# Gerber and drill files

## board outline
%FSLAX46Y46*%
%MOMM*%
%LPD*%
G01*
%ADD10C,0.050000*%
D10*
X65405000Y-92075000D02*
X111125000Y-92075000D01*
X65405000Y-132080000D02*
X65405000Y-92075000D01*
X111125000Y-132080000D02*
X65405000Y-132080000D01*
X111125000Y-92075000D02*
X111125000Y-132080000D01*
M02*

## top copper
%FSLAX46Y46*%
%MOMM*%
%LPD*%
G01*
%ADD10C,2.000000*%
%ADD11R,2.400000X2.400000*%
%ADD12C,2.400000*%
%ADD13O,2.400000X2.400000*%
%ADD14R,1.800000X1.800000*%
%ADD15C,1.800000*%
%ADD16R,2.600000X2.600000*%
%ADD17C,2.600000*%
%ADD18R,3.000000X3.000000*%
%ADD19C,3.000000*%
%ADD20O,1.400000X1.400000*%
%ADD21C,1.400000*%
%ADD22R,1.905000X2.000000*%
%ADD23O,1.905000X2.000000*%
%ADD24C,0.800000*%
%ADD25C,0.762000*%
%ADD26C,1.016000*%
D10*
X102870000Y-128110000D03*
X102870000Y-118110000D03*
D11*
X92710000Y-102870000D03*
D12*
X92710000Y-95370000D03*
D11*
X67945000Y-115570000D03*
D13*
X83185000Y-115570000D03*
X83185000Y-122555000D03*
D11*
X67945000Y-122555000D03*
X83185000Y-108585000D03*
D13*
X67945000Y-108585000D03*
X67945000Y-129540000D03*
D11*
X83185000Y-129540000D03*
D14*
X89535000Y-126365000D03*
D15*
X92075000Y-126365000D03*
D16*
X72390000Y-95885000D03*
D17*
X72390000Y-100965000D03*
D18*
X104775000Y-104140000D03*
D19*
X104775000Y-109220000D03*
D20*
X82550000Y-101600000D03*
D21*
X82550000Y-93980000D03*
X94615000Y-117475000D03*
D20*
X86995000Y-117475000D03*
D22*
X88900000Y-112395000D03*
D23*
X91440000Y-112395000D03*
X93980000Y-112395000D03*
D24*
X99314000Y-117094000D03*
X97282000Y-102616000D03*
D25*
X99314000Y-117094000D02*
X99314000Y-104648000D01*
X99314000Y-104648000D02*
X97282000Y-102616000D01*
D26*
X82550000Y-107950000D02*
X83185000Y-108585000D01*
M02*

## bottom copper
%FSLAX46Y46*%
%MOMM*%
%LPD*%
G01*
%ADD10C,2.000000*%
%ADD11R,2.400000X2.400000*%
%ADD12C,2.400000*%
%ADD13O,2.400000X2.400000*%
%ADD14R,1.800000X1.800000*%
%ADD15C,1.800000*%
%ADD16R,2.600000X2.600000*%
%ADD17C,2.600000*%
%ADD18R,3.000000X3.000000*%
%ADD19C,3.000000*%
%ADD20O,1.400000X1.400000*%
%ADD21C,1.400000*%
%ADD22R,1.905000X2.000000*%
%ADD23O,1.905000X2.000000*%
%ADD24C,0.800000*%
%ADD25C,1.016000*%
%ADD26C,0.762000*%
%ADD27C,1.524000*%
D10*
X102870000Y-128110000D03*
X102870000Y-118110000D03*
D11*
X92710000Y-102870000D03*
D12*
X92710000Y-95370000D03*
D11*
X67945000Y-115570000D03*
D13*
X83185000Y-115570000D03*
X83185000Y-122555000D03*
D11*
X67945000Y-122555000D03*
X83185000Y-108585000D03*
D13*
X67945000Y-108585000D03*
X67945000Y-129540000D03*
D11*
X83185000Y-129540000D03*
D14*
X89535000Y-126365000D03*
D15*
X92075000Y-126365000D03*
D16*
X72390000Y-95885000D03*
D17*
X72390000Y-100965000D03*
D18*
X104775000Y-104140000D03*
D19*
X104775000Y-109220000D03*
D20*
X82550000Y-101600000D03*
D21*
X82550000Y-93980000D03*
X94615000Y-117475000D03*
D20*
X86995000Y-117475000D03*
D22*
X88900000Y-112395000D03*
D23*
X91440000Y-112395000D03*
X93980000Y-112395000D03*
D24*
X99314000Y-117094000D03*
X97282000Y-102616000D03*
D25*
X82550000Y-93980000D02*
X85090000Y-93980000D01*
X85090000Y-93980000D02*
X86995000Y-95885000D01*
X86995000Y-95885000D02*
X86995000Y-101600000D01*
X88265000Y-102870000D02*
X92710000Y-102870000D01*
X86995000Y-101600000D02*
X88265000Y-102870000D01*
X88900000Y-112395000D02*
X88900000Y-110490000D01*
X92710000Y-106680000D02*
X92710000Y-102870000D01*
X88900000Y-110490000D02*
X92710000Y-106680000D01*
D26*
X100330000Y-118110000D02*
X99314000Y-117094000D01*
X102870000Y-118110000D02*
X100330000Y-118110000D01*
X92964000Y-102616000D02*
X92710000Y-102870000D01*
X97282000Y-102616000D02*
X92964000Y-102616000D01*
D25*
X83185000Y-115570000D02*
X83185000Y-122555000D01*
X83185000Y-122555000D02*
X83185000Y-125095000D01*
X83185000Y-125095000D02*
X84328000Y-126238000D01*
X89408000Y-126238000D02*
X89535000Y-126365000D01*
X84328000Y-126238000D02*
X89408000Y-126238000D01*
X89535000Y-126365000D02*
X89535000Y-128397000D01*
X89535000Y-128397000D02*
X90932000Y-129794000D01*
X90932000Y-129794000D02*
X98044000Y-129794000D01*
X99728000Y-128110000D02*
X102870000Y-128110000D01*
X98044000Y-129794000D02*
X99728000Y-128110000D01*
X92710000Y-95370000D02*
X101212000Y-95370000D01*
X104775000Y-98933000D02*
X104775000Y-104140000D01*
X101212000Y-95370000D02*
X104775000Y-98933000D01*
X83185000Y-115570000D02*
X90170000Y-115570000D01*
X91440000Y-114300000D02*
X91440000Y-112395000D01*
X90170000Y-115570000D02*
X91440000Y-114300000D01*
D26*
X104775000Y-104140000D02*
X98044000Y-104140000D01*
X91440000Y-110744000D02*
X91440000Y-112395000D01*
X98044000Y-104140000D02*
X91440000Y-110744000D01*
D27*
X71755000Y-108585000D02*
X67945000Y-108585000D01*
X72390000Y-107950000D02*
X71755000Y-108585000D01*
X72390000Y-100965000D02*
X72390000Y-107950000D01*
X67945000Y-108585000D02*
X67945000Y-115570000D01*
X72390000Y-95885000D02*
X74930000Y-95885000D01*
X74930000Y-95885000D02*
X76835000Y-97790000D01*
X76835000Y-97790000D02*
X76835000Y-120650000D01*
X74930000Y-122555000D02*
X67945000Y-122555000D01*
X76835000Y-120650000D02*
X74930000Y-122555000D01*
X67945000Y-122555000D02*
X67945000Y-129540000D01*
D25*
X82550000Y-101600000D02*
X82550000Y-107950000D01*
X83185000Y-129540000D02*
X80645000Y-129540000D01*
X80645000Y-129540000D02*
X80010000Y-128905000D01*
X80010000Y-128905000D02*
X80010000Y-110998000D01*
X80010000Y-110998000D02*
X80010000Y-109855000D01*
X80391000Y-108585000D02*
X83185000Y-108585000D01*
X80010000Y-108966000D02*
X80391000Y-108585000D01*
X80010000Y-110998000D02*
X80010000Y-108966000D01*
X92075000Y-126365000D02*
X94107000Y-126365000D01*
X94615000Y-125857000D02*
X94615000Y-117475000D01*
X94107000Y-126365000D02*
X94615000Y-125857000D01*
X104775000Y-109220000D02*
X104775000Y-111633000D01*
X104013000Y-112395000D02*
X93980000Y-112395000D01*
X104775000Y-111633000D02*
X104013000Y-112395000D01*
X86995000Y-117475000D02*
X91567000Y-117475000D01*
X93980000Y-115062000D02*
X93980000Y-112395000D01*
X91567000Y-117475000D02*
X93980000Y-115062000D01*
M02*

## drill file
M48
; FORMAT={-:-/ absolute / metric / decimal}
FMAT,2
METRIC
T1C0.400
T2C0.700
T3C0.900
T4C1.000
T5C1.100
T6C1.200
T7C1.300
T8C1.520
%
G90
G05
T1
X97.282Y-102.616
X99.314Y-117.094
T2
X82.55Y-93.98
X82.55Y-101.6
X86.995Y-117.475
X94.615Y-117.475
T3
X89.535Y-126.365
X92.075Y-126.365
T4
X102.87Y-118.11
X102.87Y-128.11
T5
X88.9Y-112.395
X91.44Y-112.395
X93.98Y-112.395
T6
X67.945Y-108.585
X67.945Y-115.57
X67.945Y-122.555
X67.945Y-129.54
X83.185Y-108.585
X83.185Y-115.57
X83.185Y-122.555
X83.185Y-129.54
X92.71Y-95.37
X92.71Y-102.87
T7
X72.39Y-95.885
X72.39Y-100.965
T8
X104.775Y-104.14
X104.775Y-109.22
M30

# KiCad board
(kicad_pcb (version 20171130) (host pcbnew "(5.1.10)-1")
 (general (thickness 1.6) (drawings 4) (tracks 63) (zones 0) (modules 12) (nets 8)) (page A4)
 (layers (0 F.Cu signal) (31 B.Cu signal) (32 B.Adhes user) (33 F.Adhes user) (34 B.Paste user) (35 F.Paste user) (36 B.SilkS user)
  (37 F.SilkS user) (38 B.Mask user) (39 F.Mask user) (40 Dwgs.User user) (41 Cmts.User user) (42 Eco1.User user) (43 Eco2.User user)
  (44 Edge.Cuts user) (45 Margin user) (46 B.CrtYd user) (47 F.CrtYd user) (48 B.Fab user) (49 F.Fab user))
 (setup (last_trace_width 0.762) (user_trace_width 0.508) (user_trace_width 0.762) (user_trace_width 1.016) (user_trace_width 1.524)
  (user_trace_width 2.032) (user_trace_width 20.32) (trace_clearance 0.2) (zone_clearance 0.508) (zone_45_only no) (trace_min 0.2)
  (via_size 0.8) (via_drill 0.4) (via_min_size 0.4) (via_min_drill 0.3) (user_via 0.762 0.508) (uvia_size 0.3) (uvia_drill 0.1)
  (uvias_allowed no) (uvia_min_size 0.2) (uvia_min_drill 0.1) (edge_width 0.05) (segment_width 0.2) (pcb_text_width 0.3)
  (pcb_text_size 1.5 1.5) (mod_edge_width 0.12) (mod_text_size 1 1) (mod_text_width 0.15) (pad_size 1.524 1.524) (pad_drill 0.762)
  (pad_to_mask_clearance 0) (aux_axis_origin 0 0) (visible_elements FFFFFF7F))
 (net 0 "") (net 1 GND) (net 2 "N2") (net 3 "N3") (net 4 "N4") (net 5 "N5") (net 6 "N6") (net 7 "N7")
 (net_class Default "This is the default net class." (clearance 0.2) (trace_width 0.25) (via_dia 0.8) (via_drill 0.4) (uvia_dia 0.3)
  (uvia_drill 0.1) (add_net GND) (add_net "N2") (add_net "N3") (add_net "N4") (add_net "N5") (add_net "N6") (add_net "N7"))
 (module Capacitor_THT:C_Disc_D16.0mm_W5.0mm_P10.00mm (layer F.Cu) (at 102.87 118.11 270)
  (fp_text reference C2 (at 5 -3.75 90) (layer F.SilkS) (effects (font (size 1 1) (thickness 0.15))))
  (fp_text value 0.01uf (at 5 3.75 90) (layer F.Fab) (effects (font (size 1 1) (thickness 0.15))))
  (pad 2 thru_hole circle (at 10 0 270) (size 2 2) (drill 1) (layers *.Cu *.Mask) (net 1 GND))
  (pad 1 thru_hole circle (at 0 0 270) (size 2 2) (drill 1) (layers *.Cu *.Mask) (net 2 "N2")))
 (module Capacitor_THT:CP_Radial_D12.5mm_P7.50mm (layer F.Cu) (at 92.71 102.87 90)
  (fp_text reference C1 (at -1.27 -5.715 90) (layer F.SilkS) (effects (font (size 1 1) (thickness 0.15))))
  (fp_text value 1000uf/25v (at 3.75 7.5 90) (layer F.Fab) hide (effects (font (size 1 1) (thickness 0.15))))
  (pad 1 thru_hole rect (at 0 0 90) (size 2.4 2.4) (drill 1.2) (layers *.Cu *.Mask) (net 2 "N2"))
  (pad 2 thru_hole circle (at 7.5 0 90) (size 2.4 2.4) (drill 1.2) (layers *.Cu *.Mask) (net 1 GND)))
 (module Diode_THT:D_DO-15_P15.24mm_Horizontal (layer F.Cu) (at 67.945 115.57)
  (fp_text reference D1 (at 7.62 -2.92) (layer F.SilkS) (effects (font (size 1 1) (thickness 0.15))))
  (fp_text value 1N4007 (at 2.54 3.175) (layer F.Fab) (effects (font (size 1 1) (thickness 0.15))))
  (pad 1 thru_hole rect (at 0 0) (size 2.4 2.4) (drill 1.2) (layers *.Cu *.Mask) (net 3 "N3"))
  (pad 2 thru_hole oval (at 15.24 0) (size 2.4 2.4) (drill 1.2) (layers *.Cu *.Mask) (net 1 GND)))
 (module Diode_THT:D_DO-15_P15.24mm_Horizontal (layer F.Cu) (at 67.945 122.555)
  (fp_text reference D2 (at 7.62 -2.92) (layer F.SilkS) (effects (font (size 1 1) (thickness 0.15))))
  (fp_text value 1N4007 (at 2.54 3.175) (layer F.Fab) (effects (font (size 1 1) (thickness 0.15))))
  (pad 2 thru_hole oval (at 15.24 0) (size 2.4 2.4) (drill 1.2) (layers *.Cu *.Mask) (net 1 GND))
  (pad 1 thru_hole rect (at 0 0) (size 2.4 2.4) (drill 1.2) (layers *.Cu *.Mask) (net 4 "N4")))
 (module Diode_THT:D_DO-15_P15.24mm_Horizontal (layer F.Cu) (at 83.185 108.585 180)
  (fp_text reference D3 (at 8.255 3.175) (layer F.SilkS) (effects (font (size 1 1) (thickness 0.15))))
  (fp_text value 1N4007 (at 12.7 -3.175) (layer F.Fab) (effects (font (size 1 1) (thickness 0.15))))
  (pad 1 thru_hole rect (at 0 0 180) (size 2.4 2.4) (drill 1.2) (layers *.Cu *.Mask) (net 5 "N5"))
  (pad 2 thru_hole oval (at 15.24 0 180) (size 2.4 2.4) (drill 1.2) (layers *.Cu *.Mask) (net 3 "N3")))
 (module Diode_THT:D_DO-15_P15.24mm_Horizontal (layer F.Cu) (at 83.185 129.54 180)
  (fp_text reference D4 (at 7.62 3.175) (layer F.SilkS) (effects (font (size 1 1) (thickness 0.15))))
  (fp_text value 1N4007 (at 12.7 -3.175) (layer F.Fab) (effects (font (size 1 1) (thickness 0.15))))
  (pad 2 thru_hole oval (at 15.24 0 180) (size 2.4 2.4) (drill 1.2) (layers *.Cu *.Mask) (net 4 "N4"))
  (pad 1 thru_hole rect (at 0 0 180) (size 2.4 2.4) (drill 1.2) (layers *.Cu *.Mask) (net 5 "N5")))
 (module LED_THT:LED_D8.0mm (layer F.Cu) (at 89.535 126.365)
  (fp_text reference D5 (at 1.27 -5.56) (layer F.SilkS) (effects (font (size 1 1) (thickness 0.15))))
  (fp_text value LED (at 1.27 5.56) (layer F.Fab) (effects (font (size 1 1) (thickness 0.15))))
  (pad 1 thru_hole rect (at 0 0) (size 1.8 1.8) (drill 0.9) (layers *.Cu *.Mask) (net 1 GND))
  (pad 2 thru_hole circle (at 2.54 0) (size 1.8 1.8) (drill 0.9) (layers *.Cu *.Mask) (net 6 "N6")))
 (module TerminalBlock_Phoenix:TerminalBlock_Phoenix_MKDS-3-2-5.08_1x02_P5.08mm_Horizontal (layer F.Cu) (at 72.39 95.885 270)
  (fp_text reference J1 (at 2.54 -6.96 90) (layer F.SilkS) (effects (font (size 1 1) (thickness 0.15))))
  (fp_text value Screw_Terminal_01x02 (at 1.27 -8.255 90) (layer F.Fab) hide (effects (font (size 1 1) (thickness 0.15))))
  (pad 1 thru_hole rect (at 0 0 270) (size 2.6 2.6) (drill 1.3) (layers *.Cu *.Mask) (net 4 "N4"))
  (pad 2 thru_hole circle (at 5.08 0 270) (size 2.6 2.6) (drill 1.3) (layers *.Cu *.Mask) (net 3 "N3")))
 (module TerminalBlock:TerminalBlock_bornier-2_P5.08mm (layer F.Cu) (at 104.775 104.14 270)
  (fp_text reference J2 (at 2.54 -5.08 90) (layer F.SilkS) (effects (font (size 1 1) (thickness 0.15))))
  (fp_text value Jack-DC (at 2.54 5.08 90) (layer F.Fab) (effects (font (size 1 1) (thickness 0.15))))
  (pad 1 thru_hole rect (at 0 0 270) (size 3 3) (drill 1.52) (layers *.Cu *.Mask) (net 1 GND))
  (pad 2 thru_hole circle (at 5.08 0 270) (size 3 3) (drill 1.52) (layers *.Cu *.Mask) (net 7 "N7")))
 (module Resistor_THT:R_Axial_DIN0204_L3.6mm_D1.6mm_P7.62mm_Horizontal (layer F.Cu) (at 82.55 93.98 270)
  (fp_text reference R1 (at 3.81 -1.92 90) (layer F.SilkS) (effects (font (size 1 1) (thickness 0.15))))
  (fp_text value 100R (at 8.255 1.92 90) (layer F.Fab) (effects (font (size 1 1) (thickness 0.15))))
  (pad 2 thru_hole oval (at 7.62 0 270) (size 1.4 1.4) (drill 0.7) (layers *.Cu *.Mask) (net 5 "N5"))
  (pad 1 thru_hole circle (at 0 0 270) (size 1.4 1.4) (drill 0.7) (layers *.Cu *.Mask) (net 2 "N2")))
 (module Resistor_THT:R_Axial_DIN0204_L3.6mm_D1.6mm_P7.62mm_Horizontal (layer F.Cu) (at 94.615 117.475 180)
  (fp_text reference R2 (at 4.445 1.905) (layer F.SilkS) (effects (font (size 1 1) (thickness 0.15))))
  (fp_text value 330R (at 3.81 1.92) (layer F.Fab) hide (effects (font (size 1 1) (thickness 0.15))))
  (pad 1 thru_hole circle (at 0 0 180) (size 1.4 1.4) (drill 0.7) (layers *.Cu *.Mask) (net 6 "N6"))
  (pad 2 thru_hole oval (at 7.62 0 180) (size 1.4 1.4) (drill 0.7) (layers *.Cu *.Mask) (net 7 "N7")))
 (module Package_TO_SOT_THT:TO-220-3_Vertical (layer F.Cu) (at 88.9 112.395)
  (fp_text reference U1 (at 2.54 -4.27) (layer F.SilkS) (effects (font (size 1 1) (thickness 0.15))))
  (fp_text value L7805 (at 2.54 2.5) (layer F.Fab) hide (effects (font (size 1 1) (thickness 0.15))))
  (pad 1 thru_hole rect (at 0 0) (size 1.905 2) (drill 1.1) (layers *.Cu *.Mask) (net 2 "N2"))
  (pad 2 thru_hole oval (at 2.54 0) (size 1.905 2) (drill 1.1) (layers *.Cu *.Mask) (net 1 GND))
  (pad 3 thru_hole oval (at 5.08 0) (size 1.905 2) (drill 1.1) (layers *.Cu *.Mask) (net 7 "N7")))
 (gr_line (start 65.405 92.075) (end 111.125 92.075) (layer Edge.Cuts) (width 0.05))
 (gr_line (start 65.405 132.08) (end 65.405 92.075) (layer Edge.Cuts) (width 0.05))
 (gr_line (start 111.125 132.08) (end 65.405 132.08) (layer Edge.Cuts) (width 0.05))
 (gr_line (start 111.125 92.075) (end 111.125 132.08) (layer Edge.Cuts) (width 0.05))
 (segment (start 82.55 93.98) (end 85.09 93.98) (width 1.016) (layer B.Cu) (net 2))
 (segment (start 85.09 93.98) (end 86.995 95.885) (width 1.016) (layer B.Cu) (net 2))
 (segment (start 86.995 95.885) (end 86.995 101.6) (width 1.016) (layer B.Cu) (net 2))
 (segment (start 88.265 102.87) (end 92.71 102.87) (width 1.016) (layer B.Cu) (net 2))
 (segment (start 86.995 101.6) (end 88.265 102.87) (width 1.016) (layer B.Cu) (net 2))
 (segment (start 88.9 112.395) (end 88.9 110.49) (width 1.016) (layer B.Cu) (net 2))
 (segment (start 92.71 106.68) (end 92.71 102.87) (width 1.016) (layer B.Cu) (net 2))
 (segment (start 88.9 110.49) (end 92.71 106.68) (width 1.016) (layer B.Cu) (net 2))
 (via (at 99.314 117.094) (size 0.8) (drill 0.4) (layers F.Cu B.Cu) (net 2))
 (segment (start 100.33 118.11) (end 99.314 117.094) (width 0.762) (layer B.Cu) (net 2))
 (segment (start 102.87 118.11) (end 100.33 118.11) (width 0.762) (layer B.Cu) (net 2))
 (segment (start 99.314 117.094) (end 99.314 104.648) (width 0.762) (layer F.Cu) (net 2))
 (via (at 97.282 102.616) (size 0.8) (drill 0.4) (layers F.Cu B.Cu) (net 2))
 (segment (start 99.314 104.648) (end 97.282 102.616) (width 0.762) (layer F.Cu) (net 2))
 (segment (start 92.964 102.616) (end 92.71 102.87) (width 0.762) (layer B.Cu) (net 2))
 (segment (start 97.282 102.616) (end 92.964 102.616) (width 0.762) (layer B.Cu) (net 2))
 (segment (start 83.185 115.57) (end 83.185 122.555) (width 1.016) (layer B.Cu) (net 1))
 (segment (start 83.185 122.555) (end 83.185 125.095) (width 1.016) (layer B.Cu) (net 1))
 (segment (start 83.185 125.095) (end 84.328 126.238) (width 1.016) (layer B.Cu) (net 1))
 (segment (start 89.408 126.238) (end 89.535 126.365) (width 1.016) (layer B.Cu) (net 1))
 (segment (start 84.328 126.238) (end 89.408 126.238) (width 1.016) (layer B.Cu) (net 1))
 (segment (start 89.535 126.365) (end 89.535 128.397) (width 1.016) (layer B.Cu) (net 1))
 (segment (start 89.535 128.397) (end 90.932 129.794) (width 1.016) (layer B.Cu) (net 1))
 (segment (start 90.932 129.794) (end 98.044 129.794) (width 1.016) (layer B.Cu) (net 1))
 (segment (start 99.728 128.11) (end 102.87 128.11) (width 1.016) (layer B.Cu) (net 1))
 (segment (start 98.044 129.794) (end 99.728 128.11) (width 1.016) (layer B.Cu) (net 1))
 (segment (start 92.71 95.37) (end 101.212 95.37) (width 1.016) (layer B.Cu) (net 1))
 (segment (start 104.775 98.933) (end 104.775 104.14) (width 1.016) (layer B.Cu) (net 1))
 (segment (start 101.212 95.37) (end 104.775 98.933) (width 1.016) (layer B.Cu) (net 1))
 (segment (start 83.185 115.57) (end 90.17 115.57) (width 1.016) (layer B.Cu) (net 1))
 (segment (start 91.44 114.3) (end 91.44 112.395) (width 1.016) (layer B.Cu) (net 1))
 (segment (start 90.17 115.57) (end 91.44 114.3) (width 1.016) (layer B.Cu) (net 1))
 (segment (start 104.775 104.14) (end 98.044 104.14) (width 0.762) (layer B.Cu) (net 1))
 (segment (start 91.44 110.744) (end 91.44 112.395) (width 0.762) (layer B.Cu) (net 1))
 (segment (start 98.044 104.14) (end 91.44 110.744) (width 0.762) (layer B.Cu) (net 1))
 (segment (start 71.755 108.585) (end 67.945 108.585) (width 1.524) (layer B.Cu) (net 3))
 (segment (start 72.39 107.95) (end 71.755 108.585) (width 1.524) (layer B.Cu) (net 3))
 (segment (start 72.39 100.965) (end 72.39 107.95) (width 1.524) (layer B.Cu) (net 3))
 (segment (start 67.945 108.585) (end 67.945 115.57) (width 1.524) (layer B.Cu) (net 3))
 (segment (start 72.39 95.885) (end 74.93 95.885) (width 1.524) (layer B.Cu) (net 4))
 (segment (start 74.93 95.885) (end 76.835 97.79) (width 1.524) (layer B.Cu) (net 4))
 (segment (start 76.835 97.79) (end 76.835 120.65) (width 1.524) (layer B.Cu) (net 4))
 (segment (start 74.93 122.555) (end 67.945 122.555) (width 1.524) (layer B.Cu) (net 4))
 (segment (start 76.835 120.65) (end 74.93 122.555) (width 1.524) (layer B.Cu) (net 4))
 (segment (start 67.945 122.555) (end 67.945 129.54) (width 1.524) (layer B.Cu) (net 4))
 (segment (start 82.55 107.95) (end 83.185 108.585) (width 1.016) (layer F.Cu) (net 5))
 (segment (start 82.55 101.6) (end 82.55 107.95) (width 1.016) (layer B.Cu) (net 5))
 (segment (start 83.185 129.54) (end 80.645 129.54) (width 1.016) (layer B.Cu) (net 5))
 (segment (start 80.645 129.54) (end 80.01 128.905) (width 1.016) (layer B.Cu) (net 5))
 (segment (start 80.01 128.905) (end 80.01 110.998) (width 1.016) (layer B.Cu) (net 5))
 (segment (start 80.01 110.998) (end 80.01 109.855) (width 1.016) (layer B.Cu) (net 5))
 (segment (start 80.391 108.585) (end 83.185 108.585) (width 1.016) (layer B.Cu) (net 5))
 (segment (start 80.01 108.966) (end 80.391 108.585) (width 1.016) (layer B.Cu) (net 5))
 (segment (start 80.01 110.998) (end 80.01 108.966) (width 1.016) (layer B.Cu) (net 5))
 (segment (start 92.075 126.365) (end 94.107 126.365) (width 1.016) (layer B.Cu) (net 6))
 (segment (start 94.615 125.857) (end 94.615 117.475) (width 1.016) (layer B.Cu) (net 6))
 (segment (start 94.107 126.365) (end 94.615 125.857) (width 1.016) (layer B.Cu) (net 6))
 (segment (start 104.775 109.22) (end 104.775 111.633) (width 1.016) (layer B.Cu) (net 7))
 (segment (start 104.013 112.395) (end 93.98 112.395) (width 1.016) (layer B.Cu) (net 7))
 (segment (start 104.775 111.633) (end 104.013 112.395) (width 1.016) (layer B.Cu) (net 7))
 (segment (start 86.995 117.475) (end 91.567 117.475) (width 1.016) (layer B.Cu) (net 7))
 (segment (start 93.98 115.062) (end 93.98 112.395) (width 1.016) (layer B.Cu) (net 7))
 (segment (start 91.567 117.475) (end 93.98 115.062) (width 1.016) (layer B.Cu) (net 7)))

